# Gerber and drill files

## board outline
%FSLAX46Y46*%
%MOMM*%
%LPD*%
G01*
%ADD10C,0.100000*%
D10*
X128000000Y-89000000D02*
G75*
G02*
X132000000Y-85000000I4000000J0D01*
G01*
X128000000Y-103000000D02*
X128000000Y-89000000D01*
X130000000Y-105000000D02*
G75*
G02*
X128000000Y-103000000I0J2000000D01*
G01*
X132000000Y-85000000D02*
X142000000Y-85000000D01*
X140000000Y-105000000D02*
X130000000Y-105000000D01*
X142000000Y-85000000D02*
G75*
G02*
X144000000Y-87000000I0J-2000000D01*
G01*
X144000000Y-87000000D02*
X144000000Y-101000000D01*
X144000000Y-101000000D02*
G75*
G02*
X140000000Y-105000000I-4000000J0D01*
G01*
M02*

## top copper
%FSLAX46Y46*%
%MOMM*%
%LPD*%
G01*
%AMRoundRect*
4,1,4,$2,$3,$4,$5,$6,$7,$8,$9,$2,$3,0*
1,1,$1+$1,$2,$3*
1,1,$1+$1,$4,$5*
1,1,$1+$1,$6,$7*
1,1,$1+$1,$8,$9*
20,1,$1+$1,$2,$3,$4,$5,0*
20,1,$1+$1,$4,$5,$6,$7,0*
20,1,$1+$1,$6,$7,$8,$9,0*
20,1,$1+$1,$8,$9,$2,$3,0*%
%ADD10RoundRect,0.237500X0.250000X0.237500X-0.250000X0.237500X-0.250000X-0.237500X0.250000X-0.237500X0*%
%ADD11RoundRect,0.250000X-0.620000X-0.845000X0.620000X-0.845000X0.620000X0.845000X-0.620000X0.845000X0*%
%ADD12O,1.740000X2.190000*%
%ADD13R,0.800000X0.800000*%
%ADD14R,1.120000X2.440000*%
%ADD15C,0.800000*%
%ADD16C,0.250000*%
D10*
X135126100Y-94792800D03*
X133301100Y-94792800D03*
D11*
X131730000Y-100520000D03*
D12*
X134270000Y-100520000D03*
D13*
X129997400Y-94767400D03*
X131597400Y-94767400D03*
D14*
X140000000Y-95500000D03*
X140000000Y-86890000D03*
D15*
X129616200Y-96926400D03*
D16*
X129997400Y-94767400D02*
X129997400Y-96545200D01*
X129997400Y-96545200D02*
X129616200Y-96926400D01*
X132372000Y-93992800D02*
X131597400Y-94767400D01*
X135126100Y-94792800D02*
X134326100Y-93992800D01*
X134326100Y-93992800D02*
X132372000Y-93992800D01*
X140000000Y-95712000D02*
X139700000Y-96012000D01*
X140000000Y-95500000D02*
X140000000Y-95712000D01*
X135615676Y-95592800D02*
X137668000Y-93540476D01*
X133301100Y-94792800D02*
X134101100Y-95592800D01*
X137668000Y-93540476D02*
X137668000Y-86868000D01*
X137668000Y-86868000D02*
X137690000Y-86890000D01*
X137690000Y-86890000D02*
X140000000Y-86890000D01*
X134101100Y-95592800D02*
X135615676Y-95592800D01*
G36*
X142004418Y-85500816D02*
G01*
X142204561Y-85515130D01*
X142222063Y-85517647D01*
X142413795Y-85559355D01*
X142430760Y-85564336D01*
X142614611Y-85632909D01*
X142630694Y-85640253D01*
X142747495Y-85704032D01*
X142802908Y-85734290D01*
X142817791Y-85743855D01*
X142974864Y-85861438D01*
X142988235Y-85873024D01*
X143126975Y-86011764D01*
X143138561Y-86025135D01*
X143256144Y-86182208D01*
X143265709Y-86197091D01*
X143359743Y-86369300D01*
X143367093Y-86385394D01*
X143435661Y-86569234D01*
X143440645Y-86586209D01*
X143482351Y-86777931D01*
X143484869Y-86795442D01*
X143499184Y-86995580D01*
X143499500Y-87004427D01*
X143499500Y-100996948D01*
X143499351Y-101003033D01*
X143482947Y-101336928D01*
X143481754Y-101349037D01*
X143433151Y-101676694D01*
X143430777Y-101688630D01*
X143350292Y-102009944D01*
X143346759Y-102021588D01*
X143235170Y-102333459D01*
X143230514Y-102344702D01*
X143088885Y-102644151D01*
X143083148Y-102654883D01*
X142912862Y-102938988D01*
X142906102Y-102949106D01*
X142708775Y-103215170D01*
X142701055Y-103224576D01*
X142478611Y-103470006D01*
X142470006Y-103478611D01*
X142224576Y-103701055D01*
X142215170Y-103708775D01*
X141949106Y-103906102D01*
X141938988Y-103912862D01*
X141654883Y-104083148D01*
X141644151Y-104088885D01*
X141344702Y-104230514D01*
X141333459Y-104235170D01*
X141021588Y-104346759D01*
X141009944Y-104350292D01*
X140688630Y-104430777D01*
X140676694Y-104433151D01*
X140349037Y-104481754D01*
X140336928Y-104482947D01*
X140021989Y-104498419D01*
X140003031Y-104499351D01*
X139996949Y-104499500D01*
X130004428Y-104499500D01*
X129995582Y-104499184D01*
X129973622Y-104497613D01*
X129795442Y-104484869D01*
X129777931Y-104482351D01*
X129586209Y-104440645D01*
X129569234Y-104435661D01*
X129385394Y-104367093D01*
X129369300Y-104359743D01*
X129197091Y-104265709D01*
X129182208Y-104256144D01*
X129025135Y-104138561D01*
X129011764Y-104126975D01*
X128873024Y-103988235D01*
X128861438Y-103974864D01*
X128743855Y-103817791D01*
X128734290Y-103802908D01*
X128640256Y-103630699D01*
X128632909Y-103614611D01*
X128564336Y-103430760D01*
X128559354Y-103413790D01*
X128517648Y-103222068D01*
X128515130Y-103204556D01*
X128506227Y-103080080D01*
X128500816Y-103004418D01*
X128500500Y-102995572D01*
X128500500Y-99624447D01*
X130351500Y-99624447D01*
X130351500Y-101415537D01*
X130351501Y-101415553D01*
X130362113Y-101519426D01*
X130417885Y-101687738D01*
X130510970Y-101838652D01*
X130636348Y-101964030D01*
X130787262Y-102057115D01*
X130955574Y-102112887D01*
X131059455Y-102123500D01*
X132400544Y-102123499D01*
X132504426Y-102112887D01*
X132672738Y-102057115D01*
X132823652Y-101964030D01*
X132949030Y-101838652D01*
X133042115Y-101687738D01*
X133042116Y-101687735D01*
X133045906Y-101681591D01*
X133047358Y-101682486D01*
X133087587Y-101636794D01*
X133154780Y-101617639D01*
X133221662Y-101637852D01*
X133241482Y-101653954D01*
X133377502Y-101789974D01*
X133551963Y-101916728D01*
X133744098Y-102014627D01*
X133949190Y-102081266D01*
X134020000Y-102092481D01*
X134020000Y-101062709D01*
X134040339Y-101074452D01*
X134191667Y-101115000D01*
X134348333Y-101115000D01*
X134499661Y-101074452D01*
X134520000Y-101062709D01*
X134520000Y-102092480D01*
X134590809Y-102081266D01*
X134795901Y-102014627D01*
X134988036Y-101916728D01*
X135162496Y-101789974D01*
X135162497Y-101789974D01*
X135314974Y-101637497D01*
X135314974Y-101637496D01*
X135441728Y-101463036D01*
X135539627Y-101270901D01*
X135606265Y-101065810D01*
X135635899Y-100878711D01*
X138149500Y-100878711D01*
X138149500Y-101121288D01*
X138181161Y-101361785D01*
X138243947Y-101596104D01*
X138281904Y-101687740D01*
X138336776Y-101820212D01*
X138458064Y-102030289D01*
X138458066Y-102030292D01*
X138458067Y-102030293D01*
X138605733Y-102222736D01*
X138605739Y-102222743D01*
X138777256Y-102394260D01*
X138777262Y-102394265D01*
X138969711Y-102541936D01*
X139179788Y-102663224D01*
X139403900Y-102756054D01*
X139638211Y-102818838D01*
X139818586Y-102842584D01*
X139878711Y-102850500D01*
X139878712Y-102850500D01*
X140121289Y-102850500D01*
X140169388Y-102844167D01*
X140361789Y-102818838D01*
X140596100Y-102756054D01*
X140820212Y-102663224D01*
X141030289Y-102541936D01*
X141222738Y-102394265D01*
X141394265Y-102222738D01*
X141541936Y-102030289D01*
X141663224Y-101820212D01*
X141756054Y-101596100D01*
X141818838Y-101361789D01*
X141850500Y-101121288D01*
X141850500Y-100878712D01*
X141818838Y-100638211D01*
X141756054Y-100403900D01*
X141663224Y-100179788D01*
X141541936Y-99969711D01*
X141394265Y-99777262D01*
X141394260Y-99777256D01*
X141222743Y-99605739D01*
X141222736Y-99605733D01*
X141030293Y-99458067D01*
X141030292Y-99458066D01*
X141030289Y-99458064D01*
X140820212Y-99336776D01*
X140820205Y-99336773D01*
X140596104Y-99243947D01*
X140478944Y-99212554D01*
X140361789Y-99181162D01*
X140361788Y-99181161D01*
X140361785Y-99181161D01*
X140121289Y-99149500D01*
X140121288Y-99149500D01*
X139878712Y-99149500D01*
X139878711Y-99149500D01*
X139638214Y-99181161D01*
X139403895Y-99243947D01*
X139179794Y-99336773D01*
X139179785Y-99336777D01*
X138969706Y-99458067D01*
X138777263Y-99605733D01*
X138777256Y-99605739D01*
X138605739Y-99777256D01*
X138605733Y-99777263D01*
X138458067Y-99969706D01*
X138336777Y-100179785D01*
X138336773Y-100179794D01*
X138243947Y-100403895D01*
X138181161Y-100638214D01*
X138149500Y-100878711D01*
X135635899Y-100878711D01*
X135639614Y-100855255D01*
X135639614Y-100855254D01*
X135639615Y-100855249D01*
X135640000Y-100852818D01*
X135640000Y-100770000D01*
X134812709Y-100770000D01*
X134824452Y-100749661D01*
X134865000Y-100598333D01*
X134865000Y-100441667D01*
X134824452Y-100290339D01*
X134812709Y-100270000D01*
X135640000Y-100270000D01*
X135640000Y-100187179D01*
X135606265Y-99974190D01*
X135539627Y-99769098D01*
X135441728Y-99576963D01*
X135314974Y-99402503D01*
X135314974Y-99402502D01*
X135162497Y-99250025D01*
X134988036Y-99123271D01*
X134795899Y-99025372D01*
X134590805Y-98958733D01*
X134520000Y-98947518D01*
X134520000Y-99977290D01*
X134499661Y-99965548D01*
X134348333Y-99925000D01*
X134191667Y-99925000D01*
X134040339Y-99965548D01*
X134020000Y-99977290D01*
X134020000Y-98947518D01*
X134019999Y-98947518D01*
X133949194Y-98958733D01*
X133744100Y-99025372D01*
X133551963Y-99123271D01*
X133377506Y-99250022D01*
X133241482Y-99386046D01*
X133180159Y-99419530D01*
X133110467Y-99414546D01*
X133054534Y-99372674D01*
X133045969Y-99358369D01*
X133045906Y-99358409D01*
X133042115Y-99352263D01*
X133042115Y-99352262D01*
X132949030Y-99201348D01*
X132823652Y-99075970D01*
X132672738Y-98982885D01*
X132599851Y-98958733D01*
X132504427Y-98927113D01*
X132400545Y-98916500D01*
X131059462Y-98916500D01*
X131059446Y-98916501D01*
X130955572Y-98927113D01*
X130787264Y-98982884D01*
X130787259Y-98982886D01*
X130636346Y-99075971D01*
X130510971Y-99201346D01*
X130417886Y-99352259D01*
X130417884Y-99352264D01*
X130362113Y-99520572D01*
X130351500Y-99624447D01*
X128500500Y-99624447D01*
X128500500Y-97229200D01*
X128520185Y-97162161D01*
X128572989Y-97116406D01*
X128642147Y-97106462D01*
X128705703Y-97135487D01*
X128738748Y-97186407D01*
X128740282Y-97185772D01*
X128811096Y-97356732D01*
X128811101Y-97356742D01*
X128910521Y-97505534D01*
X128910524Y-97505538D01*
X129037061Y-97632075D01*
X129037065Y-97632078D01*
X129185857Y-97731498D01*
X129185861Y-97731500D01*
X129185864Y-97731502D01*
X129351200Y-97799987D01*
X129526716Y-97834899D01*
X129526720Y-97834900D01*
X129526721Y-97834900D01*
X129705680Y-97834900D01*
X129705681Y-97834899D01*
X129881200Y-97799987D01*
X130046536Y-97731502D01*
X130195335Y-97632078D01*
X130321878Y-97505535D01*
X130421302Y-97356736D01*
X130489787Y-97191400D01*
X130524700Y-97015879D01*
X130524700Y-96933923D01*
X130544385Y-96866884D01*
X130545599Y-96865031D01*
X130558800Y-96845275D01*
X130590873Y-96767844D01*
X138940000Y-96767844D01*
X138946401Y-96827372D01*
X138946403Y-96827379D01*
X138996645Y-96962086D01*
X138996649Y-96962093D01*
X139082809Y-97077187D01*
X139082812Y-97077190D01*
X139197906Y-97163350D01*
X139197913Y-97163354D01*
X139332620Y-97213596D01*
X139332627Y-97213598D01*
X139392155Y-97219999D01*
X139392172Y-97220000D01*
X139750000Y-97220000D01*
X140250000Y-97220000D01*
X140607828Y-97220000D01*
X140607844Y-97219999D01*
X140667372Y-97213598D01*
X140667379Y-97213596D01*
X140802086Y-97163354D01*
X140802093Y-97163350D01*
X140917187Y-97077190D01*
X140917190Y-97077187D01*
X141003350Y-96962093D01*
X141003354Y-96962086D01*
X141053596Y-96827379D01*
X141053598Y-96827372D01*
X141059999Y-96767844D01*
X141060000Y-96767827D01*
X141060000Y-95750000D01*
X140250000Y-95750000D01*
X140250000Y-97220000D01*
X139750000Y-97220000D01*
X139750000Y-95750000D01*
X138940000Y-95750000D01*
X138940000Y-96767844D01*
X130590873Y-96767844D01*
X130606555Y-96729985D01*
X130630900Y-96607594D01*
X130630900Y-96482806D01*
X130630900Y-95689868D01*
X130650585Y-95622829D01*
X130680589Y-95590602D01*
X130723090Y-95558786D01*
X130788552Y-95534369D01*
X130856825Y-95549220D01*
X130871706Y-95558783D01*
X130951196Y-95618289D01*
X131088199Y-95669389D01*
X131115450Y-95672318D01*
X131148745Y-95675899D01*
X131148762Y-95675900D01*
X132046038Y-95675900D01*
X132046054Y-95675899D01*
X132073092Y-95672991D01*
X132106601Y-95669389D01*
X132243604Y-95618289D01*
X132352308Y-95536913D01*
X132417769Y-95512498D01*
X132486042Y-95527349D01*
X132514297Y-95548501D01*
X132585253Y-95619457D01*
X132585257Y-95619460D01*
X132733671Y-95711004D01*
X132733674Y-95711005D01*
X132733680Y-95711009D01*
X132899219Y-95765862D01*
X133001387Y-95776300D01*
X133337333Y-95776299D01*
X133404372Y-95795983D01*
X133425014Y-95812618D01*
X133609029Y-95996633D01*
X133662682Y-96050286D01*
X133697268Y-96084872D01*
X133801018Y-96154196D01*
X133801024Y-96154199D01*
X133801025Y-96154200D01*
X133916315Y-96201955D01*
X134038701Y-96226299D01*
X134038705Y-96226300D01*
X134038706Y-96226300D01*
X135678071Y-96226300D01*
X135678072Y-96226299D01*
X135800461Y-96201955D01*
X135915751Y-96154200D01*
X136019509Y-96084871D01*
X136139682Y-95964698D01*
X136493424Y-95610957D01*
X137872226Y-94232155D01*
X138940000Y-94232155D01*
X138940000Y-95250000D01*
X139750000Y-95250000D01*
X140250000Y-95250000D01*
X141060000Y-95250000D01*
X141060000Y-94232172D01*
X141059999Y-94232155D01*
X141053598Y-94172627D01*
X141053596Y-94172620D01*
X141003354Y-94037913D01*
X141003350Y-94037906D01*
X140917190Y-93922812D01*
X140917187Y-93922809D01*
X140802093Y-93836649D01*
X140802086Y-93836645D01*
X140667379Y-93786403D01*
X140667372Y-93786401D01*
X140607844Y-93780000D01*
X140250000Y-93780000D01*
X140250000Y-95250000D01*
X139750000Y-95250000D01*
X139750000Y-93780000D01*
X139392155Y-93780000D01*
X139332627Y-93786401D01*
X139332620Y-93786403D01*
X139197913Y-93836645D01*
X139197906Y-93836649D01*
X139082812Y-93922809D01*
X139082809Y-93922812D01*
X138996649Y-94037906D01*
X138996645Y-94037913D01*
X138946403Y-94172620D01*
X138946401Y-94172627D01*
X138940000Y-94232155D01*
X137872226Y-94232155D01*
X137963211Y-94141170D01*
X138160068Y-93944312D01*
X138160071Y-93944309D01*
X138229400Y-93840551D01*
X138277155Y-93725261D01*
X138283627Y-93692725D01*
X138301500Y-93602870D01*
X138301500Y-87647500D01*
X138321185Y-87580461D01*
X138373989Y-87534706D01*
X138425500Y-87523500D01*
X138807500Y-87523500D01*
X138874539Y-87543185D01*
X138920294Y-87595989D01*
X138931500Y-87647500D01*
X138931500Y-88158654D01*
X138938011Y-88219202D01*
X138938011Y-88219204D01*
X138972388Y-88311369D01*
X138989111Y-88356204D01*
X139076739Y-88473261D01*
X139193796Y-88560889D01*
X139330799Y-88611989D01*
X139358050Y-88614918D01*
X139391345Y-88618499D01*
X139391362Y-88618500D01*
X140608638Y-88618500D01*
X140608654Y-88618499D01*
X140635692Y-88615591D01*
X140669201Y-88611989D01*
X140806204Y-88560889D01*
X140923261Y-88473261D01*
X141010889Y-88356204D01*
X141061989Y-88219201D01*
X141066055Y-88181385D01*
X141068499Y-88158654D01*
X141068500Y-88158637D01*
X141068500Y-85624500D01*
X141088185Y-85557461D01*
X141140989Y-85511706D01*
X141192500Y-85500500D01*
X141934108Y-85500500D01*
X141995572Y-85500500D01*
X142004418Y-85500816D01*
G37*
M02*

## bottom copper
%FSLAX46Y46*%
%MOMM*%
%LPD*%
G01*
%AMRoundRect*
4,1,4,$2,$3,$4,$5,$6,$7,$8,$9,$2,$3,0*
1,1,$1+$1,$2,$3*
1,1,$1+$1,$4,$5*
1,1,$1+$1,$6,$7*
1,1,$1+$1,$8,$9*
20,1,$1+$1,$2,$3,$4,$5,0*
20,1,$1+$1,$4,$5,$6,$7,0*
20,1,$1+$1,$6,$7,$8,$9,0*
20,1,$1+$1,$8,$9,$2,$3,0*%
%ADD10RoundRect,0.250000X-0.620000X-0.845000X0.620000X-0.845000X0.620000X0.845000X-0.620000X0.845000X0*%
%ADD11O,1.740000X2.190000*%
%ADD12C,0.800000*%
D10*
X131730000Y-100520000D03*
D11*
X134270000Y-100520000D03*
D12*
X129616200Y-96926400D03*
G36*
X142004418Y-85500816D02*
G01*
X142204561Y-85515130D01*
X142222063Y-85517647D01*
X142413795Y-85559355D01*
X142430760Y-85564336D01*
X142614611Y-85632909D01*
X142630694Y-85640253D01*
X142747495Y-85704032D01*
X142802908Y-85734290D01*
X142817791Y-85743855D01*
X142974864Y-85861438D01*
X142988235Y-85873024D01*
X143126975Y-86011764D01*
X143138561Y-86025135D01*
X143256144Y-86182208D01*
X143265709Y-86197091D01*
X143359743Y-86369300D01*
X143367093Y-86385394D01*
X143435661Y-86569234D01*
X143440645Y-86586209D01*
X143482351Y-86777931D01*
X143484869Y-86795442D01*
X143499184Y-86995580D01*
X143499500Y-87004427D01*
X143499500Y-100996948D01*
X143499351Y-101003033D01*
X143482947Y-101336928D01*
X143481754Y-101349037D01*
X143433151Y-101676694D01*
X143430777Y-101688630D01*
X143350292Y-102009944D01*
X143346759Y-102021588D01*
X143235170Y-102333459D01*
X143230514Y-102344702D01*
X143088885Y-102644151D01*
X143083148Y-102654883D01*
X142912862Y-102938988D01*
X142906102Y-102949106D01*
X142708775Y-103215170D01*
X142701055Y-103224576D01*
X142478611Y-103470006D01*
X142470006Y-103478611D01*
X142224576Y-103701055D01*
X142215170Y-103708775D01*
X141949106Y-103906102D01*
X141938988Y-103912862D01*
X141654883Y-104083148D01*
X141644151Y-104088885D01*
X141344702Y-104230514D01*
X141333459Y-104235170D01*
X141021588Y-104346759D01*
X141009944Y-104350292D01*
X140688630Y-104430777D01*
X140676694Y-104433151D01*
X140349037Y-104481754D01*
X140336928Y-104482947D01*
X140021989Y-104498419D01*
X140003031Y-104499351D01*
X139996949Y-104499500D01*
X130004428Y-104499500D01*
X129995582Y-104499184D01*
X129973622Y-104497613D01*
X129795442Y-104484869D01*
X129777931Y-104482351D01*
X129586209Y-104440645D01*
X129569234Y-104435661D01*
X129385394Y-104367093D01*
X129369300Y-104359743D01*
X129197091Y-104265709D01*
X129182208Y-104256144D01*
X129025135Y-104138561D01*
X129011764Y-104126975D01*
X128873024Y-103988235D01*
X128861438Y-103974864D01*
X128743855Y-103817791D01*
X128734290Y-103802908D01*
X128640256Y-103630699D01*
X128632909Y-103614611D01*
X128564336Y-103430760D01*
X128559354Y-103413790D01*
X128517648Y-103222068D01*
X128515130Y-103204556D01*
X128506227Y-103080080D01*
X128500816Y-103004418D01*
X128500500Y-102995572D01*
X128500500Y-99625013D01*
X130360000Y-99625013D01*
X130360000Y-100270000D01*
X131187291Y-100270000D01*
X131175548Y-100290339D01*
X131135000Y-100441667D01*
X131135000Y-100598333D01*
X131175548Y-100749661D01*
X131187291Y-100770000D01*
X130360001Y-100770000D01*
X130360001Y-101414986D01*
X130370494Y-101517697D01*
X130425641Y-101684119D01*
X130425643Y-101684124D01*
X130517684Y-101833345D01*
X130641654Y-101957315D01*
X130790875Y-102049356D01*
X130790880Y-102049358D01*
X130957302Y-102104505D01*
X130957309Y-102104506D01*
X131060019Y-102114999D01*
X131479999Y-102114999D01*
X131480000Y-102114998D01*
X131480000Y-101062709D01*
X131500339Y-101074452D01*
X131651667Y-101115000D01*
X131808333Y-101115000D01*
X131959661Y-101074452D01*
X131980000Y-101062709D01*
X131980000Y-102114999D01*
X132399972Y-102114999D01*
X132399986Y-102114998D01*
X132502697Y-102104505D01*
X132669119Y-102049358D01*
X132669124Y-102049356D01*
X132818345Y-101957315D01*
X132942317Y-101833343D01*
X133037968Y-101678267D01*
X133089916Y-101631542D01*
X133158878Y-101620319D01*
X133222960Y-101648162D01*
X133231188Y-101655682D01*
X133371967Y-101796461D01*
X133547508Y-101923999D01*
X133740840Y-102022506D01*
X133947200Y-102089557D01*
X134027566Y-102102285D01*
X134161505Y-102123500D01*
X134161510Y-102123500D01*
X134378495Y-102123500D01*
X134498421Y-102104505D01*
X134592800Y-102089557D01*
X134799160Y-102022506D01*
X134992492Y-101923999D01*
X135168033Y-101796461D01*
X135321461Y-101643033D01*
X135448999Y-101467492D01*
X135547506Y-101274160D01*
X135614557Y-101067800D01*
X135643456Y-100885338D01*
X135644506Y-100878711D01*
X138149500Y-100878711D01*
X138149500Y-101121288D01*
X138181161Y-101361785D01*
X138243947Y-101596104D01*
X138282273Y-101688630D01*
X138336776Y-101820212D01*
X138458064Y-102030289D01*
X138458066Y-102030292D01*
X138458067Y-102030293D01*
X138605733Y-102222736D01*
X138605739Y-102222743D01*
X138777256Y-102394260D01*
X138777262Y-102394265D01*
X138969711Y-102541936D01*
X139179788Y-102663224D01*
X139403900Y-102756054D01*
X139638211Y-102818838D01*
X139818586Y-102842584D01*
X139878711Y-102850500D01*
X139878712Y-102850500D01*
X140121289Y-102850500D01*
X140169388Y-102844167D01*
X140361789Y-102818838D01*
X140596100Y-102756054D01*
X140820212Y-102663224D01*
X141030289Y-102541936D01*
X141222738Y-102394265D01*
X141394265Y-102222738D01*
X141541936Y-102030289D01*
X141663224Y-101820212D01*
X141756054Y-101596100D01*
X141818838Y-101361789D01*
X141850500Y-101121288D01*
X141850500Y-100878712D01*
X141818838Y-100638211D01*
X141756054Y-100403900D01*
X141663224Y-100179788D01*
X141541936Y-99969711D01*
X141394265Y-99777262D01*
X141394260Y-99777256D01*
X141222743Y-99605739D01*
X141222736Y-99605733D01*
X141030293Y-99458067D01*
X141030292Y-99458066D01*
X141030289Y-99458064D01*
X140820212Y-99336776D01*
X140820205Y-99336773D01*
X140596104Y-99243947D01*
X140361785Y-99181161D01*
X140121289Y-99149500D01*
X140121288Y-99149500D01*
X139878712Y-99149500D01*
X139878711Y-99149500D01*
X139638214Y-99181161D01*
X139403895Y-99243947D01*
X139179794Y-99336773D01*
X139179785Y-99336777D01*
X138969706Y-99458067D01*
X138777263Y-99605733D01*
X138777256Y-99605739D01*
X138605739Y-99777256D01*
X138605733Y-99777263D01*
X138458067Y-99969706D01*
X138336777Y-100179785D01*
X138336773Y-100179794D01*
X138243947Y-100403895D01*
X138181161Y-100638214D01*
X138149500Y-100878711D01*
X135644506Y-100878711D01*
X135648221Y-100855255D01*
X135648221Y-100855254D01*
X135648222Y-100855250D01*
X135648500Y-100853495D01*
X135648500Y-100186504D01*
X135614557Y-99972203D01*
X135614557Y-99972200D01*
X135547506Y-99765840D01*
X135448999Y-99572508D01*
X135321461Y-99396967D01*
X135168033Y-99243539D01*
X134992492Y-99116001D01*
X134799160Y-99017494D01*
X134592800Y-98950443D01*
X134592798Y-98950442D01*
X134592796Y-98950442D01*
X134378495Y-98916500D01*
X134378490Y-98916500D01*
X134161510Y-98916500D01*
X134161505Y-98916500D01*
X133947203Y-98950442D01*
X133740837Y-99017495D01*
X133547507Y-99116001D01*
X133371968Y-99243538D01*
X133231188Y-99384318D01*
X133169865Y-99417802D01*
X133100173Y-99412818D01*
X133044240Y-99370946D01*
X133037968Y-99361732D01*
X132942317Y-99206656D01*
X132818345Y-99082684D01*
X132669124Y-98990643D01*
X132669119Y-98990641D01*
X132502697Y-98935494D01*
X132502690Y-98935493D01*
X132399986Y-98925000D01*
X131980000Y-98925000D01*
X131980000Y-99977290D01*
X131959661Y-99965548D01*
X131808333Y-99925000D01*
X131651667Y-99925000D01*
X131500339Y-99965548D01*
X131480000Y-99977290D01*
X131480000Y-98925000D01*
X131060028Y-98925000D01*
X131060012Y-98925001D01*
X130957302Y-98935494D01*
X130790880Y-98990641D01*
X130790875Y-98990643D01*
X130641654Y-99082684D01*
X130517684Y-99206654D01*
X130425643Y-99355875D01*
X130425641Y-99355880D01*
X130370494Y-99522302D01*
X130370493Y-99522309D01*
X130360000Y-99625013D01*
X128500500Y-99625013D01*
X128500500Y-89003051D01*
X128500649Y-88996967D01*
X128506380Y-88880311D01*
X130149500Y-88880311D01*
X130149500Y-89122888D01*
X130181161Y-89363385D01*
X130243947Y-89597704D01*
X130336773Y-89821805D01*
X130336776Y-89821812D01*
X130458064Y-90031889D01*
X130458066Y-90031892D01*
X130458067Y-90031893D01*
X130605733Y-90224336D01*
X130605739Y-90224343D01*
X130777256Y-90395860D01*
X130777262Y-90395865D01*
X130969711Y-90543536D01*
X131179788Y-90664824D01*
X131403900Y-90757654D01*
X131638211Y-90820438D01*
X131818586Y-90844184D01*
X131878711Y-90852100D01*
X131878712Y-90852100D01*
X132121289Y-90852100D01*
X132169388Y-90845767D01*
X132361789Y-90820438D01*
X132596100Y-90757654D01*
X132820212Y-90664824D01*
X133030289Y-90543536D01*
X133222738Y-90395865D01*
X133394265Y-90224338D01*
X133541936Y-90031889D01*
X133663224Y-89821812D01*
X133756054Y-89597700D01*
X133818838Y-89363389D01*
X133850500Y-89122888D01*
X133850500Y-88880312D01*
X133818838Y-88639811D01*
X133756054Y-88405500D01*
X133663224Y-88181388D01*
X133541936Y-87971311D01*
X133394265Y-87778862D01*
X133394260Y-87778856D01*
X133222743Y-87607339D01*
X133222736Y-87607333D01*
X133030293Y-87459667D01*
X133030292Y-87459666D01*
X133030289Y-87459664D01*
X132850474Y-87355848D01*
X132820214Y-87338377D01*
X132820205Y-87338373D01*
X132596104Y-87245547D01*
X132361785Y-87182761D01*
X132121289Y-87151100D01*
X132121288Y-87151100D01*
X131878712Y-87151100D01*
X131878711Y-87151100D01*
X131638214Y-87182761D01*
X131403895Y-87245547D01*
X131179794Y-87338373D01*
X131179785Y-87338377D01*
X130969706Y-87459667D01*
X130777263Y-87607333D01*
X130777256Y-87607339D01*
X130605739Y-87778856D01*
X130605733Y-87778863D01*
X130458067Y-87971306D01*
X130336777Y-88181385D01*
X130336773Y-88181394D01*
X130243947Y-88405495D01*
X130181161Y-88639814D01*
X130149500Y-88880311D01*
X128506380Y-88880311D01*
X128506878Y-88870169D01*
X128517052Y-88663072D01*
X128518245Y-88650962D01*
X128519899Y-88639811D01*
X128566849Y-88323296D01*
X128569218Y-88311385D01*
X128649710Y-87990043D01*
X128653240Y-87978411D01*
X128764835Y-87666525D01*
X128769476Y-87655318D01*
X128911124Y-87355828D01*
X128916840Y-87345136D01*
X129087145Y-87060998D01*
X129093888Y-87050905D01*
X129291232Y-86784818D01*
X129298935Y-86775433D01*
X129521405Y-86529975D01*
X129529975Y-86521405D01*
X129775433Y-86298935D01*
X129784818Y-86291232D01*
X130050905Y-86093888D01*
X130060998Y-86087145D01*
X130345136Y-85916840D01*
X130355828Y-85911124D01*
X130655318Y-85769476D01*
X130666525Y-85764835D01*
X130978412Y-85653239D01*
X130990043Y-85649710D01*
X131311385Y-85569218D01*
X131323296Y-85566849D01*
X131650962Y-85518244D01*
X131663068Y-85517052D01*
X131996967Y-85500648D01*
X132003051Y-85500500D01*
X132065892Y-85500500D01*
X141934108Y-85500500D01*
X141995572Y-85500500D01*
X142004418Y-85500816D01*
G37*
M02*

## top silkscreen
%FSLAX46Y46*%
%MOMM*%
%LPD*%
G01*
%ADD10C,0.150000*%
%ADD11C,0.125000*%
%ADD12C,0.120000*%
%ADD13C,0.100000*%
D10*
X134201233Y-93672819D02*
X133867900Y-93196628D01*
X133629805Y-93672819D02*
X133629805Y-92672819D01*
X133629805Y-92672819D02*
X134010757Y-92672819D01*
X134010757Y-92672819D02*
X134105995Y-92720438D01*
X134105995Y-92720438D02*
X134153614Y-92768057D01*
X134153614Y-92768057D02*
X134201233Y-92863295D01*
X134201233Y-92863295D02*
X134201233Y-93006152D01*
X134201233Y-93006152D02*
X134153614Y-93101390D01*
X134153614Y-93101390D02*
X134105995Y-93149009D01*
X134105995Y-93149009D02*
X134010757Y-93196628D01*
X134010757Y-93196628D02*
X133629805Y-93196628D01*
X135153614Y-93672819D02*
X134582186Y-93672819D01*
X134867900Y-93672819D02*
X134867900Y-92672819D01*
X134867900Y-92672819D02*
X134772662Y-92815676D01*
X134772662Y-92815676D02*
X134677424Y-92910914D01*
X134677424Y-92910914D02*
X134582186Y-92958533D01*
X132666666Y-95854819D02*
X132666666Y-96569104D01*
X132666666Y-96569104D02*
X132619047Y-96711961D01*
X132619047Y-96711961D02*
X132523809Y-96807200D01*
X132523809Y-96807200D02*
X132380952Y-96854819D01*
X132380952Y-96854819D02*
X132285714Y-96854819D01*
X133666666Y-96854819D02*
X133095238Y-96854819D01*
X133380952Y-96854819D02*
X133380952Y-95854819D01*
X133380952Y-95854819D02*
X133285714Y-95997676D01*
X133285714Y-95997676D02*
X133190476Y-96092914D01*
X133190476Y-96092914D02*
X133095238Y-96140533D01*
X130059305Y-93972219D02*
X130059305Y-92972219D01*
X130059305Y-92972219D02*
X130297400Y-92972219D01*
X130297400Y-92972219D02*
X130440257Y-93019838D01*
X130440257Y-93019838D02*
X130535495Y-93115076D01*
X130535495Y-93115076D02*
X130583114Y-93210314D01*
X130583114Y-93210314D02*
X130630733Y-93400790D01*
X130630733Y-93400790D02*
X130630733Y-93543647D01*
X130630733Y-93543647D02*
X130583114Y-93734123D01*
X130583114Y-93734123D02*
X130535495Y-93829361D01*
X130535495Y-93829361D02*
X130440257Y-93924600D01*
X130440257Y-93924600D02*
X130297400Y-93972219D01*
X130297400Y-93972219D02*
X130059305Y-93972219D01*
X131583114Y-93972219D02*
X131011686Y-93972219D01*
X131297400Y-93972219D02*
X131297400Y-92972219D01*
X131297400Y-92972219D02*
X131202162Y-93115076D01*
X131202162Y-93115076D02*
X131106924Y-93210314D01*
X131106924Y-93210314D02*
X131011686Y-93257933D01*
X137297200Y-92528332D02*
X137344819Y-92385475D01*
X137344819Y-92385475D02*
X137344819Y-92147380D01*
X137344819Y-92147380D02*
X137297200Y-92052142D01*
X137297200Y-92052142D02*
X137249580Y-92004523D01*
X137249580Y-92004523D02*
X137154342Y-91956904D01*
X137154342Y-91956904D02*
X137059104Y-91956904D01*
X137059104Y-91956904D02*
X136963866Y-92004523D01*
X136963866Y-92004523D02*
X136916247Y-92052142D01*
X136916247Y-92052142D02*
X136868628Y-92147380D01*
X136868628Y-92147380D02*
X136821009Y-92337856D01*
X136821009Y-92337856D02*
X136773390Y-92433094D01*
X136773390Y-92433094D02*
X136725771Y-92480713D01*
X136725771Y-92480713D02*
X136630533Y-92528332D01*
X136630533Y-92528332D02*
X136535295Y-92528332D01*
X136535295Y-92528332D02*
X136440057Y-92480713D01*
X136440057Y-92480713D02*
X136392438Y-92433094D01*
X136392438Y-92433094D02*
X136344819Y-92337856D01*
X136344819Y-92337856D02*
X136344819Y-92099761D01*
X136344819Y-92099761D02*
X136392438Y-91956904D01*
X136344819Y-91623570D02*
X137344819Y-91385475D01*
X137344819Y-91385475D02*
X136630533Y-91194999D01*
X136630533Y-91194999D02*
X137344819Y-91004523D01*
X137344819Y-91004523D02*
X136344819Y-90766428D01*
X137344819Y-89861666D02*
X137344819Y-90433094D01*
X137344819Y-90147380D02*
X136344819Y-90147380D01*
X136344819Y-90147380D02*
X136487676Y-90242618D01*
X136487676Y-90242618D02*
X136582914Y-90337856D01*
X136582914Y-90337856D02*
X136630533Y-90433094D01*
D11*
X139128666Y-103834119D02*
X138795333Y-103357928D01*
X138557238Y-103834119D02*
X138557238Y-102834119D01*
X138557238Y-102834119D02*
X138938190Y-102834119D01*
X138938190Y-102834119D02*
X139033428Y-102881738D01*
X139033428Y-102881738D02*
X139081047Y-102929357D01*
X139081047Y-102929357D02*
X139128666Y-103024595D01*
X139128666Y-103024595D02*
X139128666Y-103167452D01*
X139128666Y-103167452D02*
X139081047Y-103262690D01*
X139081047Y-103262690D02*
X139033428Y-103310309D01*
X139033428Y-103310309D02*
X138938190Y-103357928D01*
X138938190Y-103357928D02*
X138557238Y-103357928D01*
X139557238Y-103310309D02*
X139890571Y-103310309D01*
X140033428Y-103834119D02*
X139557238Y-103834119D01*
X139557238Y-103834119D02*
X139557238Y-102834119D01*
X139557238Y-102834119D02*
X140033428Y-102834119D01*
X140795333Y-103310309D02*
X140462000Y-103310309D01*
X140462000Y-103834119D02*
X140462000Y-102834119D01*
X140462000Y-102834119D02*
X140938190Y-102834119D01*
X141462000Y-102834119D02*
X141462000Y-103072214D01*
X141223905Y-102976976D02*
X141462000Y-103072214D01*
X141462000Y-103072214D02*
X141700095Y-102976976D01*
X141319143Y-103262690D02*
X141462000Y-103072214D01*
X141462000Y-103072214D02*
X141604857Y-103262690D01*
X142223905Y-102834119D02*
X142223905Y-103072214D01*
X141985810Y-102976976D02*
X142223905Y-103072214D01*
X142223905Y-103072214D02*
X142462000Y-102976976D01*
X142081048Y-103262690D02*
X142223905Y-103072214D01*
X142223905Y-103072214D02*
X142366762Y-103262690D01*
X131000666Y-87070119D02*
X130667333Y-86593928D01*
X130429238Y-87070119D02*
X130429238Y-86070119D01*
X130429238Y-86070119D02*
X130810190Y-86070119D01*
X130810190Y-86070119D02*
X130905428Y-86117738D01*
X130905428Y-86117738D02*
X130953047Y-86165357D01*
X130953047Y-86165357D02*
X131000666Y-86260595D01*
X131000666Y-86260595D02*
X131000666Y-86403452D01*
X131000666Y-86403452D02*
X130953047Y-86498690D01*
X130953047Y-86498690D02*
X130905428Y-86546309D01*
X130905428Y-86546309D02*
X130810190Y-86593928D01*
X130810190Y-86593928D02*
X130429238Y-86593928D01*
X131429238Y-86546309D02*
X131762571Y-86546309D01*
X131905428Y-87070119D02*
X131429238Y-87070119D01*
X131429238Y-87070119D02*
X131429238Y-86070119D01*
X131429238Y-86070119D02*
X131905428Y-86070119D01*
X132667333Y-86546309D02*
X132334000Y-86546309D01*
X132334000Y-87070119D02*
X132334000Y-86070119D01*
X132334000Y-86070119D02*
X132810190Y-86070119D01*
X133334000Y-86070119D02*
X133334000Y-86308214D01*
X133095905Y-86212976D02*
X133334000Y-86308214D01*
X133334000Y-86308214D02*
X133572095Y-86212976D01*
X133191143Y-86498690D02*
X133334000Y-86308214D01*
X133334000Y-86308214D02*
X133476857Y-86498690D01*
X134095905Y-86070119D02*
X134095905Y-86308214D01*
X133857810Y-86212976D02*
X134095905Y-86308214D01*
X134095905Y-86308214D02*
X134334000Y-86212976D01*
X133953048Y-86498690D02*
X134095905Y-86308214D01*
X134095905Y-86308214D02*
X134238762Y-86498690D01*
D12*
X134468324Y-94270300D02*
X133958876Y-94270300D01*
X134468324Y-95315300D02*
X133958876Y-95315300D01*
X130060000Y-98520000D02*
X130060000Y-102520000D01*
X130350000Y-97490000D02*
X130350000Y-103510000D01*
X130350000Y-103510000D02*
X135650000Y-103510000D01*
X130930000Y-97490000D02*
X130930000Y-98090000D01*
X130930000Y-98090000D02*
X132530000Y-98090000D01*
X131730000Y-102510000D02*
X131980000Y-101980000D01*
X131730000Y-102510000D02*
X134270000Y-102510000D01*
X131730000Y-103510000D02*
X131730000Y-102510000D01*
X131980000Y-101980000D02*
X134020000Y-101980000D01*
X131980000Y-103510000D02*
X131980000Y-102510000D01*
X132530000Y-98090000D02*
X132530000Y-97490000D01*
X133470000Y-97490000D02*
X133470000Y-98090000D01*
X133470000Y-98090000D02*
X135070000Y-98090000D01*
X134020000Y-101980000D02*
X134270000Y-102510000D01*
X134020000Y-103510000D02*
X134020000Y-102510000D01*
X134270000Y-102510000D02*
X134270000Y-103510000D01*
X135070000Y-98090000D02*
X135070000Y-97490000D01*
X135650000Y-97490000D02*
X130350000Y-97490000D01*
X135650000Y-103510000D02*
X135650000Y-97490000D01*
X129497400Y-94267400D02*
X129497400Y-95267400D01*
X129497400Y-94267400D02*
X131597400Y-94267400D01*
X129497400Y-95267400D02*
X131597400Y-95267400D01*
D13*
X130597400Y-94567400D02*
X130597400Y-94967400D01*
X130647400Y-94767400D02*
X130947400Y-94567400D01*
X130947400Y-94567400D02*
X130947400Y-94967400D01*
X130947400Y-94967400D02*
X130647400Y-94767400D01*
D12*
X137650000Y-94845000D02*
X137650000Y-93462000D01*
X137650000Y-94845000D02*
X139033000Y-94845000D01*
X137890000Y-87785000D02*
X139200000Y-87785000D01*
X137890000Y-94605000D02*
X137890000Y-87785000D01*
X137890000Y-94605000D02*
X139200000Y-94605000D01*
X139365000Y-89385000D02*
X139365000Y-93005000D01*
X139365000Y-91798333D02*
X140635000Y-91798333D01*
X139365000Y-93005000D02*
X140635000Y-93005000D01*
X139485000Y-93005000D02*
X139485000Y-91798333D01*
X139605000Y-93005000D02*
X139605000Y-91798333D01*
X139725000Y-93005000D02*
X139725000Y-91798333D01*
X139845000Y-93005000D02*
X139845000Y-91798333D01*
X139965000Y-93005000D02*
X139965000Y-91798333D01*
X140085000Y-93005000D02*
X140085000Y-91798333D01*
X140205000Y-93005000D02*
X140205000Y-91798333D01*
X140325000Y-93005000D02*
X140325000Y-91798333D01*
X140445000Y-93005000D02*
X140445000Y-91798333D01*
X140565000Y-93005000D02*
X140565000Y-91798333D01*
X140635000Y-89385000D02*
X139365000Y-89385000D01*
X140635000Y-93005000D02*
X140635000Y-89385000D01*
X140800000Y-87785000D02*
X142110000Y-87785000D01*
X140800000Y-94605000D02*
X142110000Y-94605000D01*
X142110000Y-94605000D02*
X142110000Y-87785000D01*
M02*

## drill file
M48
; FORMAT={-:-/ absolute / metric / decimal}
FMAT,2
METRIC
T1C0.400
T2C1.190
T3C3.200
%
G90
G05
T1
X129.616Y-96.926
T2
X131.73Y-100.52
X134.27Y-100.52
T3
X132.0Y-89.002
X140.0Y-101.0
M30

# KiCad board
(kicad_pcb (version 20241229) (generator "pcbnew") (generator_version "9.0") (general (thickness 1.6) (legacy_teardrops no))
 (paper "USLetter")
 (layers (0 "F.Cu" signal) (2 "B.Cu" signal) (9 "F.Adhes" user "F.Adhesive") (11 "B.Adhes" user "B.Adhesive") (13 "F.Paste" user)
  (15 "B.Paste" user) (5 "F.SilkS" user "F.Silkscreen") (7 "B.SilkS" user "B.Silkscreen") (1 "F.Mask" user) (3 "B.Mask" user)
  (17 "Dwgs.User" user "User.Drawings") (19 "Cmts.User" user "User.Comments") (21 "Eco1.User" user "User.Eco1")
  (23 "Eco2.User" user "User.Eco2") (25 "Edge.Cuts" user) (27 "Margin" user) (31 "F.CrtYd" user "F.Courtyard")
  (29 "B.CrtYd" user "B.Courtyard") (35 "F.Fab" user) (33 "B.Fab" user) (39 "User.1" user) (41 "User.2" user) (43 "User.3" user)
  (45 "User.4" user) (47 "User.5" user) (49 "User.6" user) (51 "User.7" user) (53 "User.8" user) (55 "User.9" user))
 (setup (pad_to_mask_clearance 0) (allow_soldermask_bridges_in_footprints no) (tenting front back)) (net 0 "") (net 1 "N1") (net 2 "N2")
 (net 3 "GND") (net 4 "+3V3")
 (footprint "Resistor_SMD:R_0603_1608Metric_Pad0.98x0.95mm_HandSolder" (layer "F.Cu") (at 134.2136 94.7928 180)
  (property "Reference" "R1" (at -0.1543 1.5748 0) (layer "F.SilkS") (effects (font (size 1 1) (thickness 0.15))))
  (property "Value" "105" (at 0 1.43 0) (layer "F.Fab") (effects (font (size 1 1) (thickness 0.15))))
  (fp_line (start -0.254724 0.5225) (end 0.254724 0.5225) (stroke (width 0.12) (type solid)) (layer "F.SilkS"))
  (fp_line (start -0.254724 -0.5225) (end 0.254724 -0.5225) (stroke (width 0.12) (type solid)) (layer "F.SilkS"))
  (pad "1" smd roundrect (at -0.9125 0 180) (size 0.975 0.95) (layers "F.Cu" "F.Mask" "F.Paste") (roundrect_rratio 0.25) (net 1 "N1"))
  (pad "2" smd roundrect (at 0.9125 0 180) (size 0.975 0.95) (layers "F.Cu" "F.Mask" "F.Paste") (roundrect_rratio 0.25) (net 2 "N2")))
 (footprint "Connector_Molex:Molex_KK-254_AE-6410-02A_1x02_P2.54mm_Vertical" (layer "F.Cu") (at 131.73 100.52)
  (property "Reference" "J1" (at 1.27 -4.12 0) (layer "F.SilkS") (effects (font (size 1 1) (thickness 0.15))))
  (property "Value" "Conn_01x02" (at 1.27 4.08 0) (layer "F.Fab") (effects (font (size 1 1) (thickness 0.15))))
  (fp_line (start -1.67 -2) (end -1.67 2) (stroke (width 0.12) (type solid)) (layer "F.SilkS"))
  (fp_line (start -1.38 -3.03) (end -1.38 2.99) (stroke (width 0.12) (type solid)) (layer "F.SilkS"))
  (fp_line (start -1.38 2.99) (end 3.92 2.99) (stroke (width 0.12) (type solid)) (layer "F.SilkS"))
  (fp_line (start -0.8 -3.03) (end -0.8 -2.43) (stroke (width 0.12) (type solid)) (layer "F.SilkS"))
  (fp_line (start -0.8 -2.43) (end 0.8 -2.43) (stroke (width 0.12) (type solid)) (layer "F.SilkS"))
  (fp_line (start 0 1.99) (end 0.25 1.46) (stroke (width 0.12) (type solid)) (layer "F.SilkS"))
  (fp_line (start 0 1.99) (end 2.54 1.99) (stroke (width 0.12) (type solid)) (layer "F.SilkS"))
  (fp_line (start 0 2.99) (end 0 1.99) (stroke (width 0.12) (type solid)) (layer "F.SilkS"))
  (fp_line (start 0.25 1.46) (end 2.29 1.46) (stroke (width 0.12) (type solid)) (layer "F.SilkS"))
  (fp_line (start 0.25 2.99) (end 0.25 1.99) (stroke (width 0.12) (type solid)) (layer "F.SilkS"))
  (fp_line (start 0.8 -2.43) (end 0.8 -3.03) (stroke (width 0.12) (type solid)) (layer "F.SilkS"))
  (fp_line (start 1.74 -3.03) (end 1.74 -2.43) (stroke (width 0.12) (type solid)) (layer "F.SilkS"))
  (fp_line (start 1.74 -2.43) (end 3.34 -2.43) (stroke (width 0.12) (type solid)) (layer "F.SilkS"))
  (fp_line (start 2.29 1.46) (end 2.54 1.99) (stroke (width 0.12) (type solid)) (layer "F.SilkS"))
  (fp_line (start 2.29 2.99) (end 2.29 1.99) (stroke (width 0.12) (type solid)) (layer "F.SilkS"))
  (fp_line (start 2.54 1.99) (end 2.54 2.99) (stroke (width 0.12) (type solid)) (layer "F.SilkS"))
  (fp_line (start 3.34 -2.43) (end 3.34 -3.03) (stroke (width 0.12) (type solid)) (layer "F.SilkS"))
  (fp_line (start 3.92 -3.03) (end -1.38 -3.03) (stroke (width 0.12) (type solid)) (layer "F.SilkS"))
  (fp_line (start 3.92 2.99) (end 3.92 -3.03) (stroke (width 0.12) (type solid)) (layer "F.SilkS"))
  (pad "1" thru_hole roundrect (at 0 0) (size 1.74 2.19) (drill 1.19) (layers "*.Cu" "*.Mask") (remove_unused_layers no)
   (roundrect_rratio 0.143678) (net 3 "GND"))
  (pad "2" thru_hole oval (at 2.54 0) (size 1.74 2.19) (drill 1.19) (layers "*.Cu" "*.Mask") (remove_unused_layers no) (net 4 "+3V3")))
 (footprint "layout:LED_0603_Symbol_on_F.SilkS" (layer "F.Cu") (at 130.7974 94.7674)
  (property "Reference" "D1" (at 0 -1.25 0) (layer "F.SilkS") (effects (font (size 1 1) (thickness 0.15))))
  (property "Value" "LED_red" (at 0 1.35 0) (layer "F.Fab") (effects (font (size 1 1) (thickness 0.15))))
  (fp_line (start -1.3 -0.5) (end -1.3 0.5) (stroke (width 0.12) (type solid)) (layer "F.SilkS"))
  (fp_line (start -1.3 -0.5) (end 0.8 -0.5) (stroke (width 0.12) (type solid)) (layer "F.SilkS"))
  (fp_line (start -1.3 0.5) (end 0.8 0.5) (stroke (width 0.12) (type solid)) (layer "F.SilkS"))
  (fp_line (start -0.2 -0.2) (end -0.2 0.2) (stroke (width 0.1) (type solid)) (layer "F.SilkS"))
  (fp_line (start -0.15 0) (end 0.15 -0.2) (stroke (width 0.1) (type solid)) (layer "F.SilkS"))
  (fp_line (start 0.15 -0.2) (end 0.15 0.2) (stroke (width 0.1) (type solid)) (layer "F.SilkS"))
  (fp_line (start 0.15 0.2) (end -0.15 0) (stroke (width 0.1) (type solid)) (layer "F.SilkS"))
  (pad "1" smd rect (at -0.8 0 180) (size 0.8 0.8) (layers "F.Cu" "F.Mask" "F.Paste") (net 3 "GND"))
  (pad "2" smd rect (at 0.8 0 180) (size 0.8 0.8) (layers "F.Cu" "F.Mask" "F.Paste") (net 1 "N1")))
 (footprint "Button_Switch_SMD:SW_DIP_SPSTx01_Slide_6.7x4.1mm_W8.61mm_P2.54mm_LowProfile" (layer "F.Cu") (at 140 91.195 90)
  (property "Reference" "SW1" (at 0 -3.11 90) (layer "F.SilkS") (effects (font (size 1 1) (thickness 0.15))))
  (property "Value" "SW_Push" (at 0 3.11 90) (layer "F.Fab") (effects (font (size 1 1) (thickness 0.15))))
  (fp_line (start -3.65 -2.35) (end -2.267 -2.35) (stroke (width 0.12) (type solid)) (layer "F.SilkS"))
  (fp_line (start -3.65 -2.35) (end -3.65 -0.967) (stroke (width 0.12) (type solid)) (layer "F.SilkS"))
  (fp_line (start 3.41 -2.11) (end 3.41 -0.8) (stroke (width 0.12) (type solid)) (layer "F.SilkS"))
  (fp_line (start -3.41 -2.11) (end 3.41 -2.11) (stroke (width 0.12) (type solid)) (layer "F.SilkS"))
  (fp_line (start -3.41 -2.11) (end -3.41 -0.8) (stroke (width 0.12) (type solid)) (layer "F.SilkS"))
  (fp_line (start 1.81 -0.635) (end -1.81 -0.635) (stroke (width 0.12) (type solid)) (layer "F.SilkS"))
  (fp_line (start -0.603333 -0.635) (end -0.603333 0.635) (stroke (width 0.12) (type solid)) (layer "F.SilkS"))
  (fp_line (start -1.81 -0.635) (end -1.81 0.635) (stroke (width 0.12) (type solid)) (layer "F.SilkS"))
  (fp_line (start -1.81 -0.515) (end -0.603333 -0.515) (stroke (width 0.12) (type solid)) (layer "F.SilkS"))
  (fp_line (start -1.81 -0.395) (end -0.603333 -0.395) (stroke (width 0.12) (type solid)) (layer "F.SilkS"))
  (fp_line (start -1.81 -0.275) (end -0.603333 -0.275) (stroke (width 0.12) (type solid)) (layer "F.SilkS"))
  (fp_line (start -1.81 -0.155) (end -0.603333 -0.155) (stroke (width 0.12) (type solid)) (layer "F.SilkS"))
  (fp_line (start -1.81 -0.035) (end -0.603333 -0.035) (stroke (width 0.12) (type solid)) (layer "F.SilkS"))
  (fp_line (start -1.81 0.085) (end -0.603333 0.085) (stroke (width 0.12) (type solid)) (layer "F.SilkS"))
  (fp_line (start -1.81 0.205) (end -0.603333 0.205) (stroke (width 0.12) (type solid)) (layer "F.SilkS"))
  (fp_line (start -1.81 0.325) (end -0.603333 0.325) (stroke (width 0.12) (type solid)) (layer "F.SilkS"))
  (fp_line (start -1.81 0.445) (end -0.603333 0.445) (stroke (width 0.12) (type solid)) (layer "F.SilkS"))
  (fp_line (start -1.81 0.565) (end -0.603333 0.565) (stroke (width 0.12) (type solid)) (layer "F.SilkS"))
  (fp_line (start 1.81 0.635) (end 1.81 -0.635) (stroke (width 0.12) (type solid)) (layer "F.SilkS"))
  (fp_line (start -1.81 0.635) (end 1.81 0.635) (stroke (width 0.12) (type solid)) (layer "F.SilkS"))
  (fp_line (start 3.41 0.8) (end 3.41 2.11) (stroke (width 0.12) (type solid)) (layer "F.SilkS"))
  (fp_line (start -3.41 0.8) (end -3.41 2.11) (stroke (width 0.12) (type solid)) (layer "F.SilkS"))
  (fp_line (start -3.41 2.11) (end 3.41 2.11) (stroke (width 0.12) (type solid)) (layer "F.SilkS"))
  (pad "1" smd rect (at -4.305 0 90) (size 2.44 1.12) (layers "F.Cu" "F.Mask" "F.Paste") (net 4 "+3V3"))
  (pad "2" smd rect (at 4.305 0 90) (size 2.44 1.12) (layers "F.Cu" "F.Mask" "F.Paste") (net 2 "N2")))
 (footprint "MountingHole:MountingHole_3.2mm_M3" (layer "F.Cu") (at 140 101)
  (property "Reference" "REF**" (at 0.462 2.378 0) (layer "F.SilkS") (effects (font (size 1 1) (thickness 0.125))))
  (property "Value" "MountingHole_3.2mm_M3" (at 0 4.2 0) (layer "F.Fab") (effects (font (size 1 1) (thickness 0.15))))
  (pad "" np_thru_hole circle (at 0 0) (size 3.2 3.2) (drill 3.2) (layers "*.Cu" "*.Mask")))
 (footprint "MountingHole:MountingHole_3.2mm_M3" (layer "F.Cu") (at 132 89.0016)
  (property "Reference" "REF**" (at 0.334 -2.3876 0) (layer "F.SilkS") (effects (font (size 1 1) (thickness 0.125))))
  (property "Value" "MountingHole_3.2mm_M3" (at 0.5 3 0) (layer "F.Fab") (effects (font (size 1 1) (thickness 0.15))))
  (pad "" np_thru_hole circle (at 0 0) (size 3.2 3.2) (drill 3.2) (layers "*.Cu" "*.Mask")))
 (gr_arc (start 128 89) (mid 129.171573 86.171573) (end 132 85) (stroke (width 0.1) (type default)) (layer "Edge.Cuts"))
 (gr_line (start 128 103) (end 128 89) (stroke (width 0.1) (type default)) (layer "Edge.Cuts"))
 (gr_arc (start 130 105) (mid 128.585786 104.414214) (end 128 103) (stroke (width 0.1) (type default)) (layer "Edge.Cuts"))
 (gr_line (start 132 85) (end 142 85) (stroke (width 0.1) (type default)) (layer "Edge.Cuts"))
 (gr_line (start 140 105) (end 130 105) (stroke (width 0.1) (type default)) (layer "Edge.Cuts"))
 (gr_arc (start 142 85) (mid 143.414214 85.585786) (end 144 87) (stroke (width 0.1) (type default)) (layer "Edge.Cuts"))
 (gr_line (start 144 87) (end 144 101) (stroke (width 0.1) (type default)) (layer "Edge.Cuts"))
 (gr_arc (start 144 101) (mid 142.828427 103.828427) (end 140 105) (stroke (width 0.1) (type default)) (layer "Edge.Cuts"))
 (segment (start 129.9974 94.7674) (end 129.9974 96.5452) (width 0.25) (layer "F.Cu") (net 3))
 (segment (start 129.9974 96.5452) (end 129.6162 96.9264) (width 0.25) (layer "F.Cu") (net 3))
 (via (at 129.6162 96.9264) (size 0.8) (drill 0.4) (layers "F.Cu" "B.Cu") (free yes) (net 3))
 (segment (start 132.372 93.9928) (end 131.5974 94.7674) (width 0.25) (layer "F.Cu") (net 1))
 (segment (start 135.1261 94.7928) (end 134.3261 93.9928) (width 0.25) (layer "F.Cu") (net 1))
 (segment (start 134.3261 93.9928) (end 132.372 93.9928) (width 0.25) (layer "F.Cu") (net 1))
 (segment (start 140 95.712) (end 139.7 96.012) (width 0.25) (layer "F.Cu") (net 4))
 (segment (start 140 95.5) (end 140 95.712) (width 0.25) (layer "F.Cu") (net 4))
 (segment (start 135.615676 95.5928) (end 137.668 93.540476) (width 0.25) (layer "F.Cu") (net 2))
 (segment (start 133.3011 94.7928) (end 134.1011 95.5928) (width 0.25) (layer "F.Cu") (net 2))
 (segment (start 137.668 93.540476) (end 137.668 86.868) (width 0.25) (layer "F.Cu") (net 2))
 (segment (start 137.668 86.868) (end 137.69 86.89) (width 0.25) (layer "F.Cu") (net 2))
 (segment (start 137.69 86.89) (end 140 86.89) (width 0.25) (layer "F.Cu") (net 2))
 (segment (start 134.1011 95.5928) (end 135.615676 95.5928) (width 0.25) (layer "F.Cu") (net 2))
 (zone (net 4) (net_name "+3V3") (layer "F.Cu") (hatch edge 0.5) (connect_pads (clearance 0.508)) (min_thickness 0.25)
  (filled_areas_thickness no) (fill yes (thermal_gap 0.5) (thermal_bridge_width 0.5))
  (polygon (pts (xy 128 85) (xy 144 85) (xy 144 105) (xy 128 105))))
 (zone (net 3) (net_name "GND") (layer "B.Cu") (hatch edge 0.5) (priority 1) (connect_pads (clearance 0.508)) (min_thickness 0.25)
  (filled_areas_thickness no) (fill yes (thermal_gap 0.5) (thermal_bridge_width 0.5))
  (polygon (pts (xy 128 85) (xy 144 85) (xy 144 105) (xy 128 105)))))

